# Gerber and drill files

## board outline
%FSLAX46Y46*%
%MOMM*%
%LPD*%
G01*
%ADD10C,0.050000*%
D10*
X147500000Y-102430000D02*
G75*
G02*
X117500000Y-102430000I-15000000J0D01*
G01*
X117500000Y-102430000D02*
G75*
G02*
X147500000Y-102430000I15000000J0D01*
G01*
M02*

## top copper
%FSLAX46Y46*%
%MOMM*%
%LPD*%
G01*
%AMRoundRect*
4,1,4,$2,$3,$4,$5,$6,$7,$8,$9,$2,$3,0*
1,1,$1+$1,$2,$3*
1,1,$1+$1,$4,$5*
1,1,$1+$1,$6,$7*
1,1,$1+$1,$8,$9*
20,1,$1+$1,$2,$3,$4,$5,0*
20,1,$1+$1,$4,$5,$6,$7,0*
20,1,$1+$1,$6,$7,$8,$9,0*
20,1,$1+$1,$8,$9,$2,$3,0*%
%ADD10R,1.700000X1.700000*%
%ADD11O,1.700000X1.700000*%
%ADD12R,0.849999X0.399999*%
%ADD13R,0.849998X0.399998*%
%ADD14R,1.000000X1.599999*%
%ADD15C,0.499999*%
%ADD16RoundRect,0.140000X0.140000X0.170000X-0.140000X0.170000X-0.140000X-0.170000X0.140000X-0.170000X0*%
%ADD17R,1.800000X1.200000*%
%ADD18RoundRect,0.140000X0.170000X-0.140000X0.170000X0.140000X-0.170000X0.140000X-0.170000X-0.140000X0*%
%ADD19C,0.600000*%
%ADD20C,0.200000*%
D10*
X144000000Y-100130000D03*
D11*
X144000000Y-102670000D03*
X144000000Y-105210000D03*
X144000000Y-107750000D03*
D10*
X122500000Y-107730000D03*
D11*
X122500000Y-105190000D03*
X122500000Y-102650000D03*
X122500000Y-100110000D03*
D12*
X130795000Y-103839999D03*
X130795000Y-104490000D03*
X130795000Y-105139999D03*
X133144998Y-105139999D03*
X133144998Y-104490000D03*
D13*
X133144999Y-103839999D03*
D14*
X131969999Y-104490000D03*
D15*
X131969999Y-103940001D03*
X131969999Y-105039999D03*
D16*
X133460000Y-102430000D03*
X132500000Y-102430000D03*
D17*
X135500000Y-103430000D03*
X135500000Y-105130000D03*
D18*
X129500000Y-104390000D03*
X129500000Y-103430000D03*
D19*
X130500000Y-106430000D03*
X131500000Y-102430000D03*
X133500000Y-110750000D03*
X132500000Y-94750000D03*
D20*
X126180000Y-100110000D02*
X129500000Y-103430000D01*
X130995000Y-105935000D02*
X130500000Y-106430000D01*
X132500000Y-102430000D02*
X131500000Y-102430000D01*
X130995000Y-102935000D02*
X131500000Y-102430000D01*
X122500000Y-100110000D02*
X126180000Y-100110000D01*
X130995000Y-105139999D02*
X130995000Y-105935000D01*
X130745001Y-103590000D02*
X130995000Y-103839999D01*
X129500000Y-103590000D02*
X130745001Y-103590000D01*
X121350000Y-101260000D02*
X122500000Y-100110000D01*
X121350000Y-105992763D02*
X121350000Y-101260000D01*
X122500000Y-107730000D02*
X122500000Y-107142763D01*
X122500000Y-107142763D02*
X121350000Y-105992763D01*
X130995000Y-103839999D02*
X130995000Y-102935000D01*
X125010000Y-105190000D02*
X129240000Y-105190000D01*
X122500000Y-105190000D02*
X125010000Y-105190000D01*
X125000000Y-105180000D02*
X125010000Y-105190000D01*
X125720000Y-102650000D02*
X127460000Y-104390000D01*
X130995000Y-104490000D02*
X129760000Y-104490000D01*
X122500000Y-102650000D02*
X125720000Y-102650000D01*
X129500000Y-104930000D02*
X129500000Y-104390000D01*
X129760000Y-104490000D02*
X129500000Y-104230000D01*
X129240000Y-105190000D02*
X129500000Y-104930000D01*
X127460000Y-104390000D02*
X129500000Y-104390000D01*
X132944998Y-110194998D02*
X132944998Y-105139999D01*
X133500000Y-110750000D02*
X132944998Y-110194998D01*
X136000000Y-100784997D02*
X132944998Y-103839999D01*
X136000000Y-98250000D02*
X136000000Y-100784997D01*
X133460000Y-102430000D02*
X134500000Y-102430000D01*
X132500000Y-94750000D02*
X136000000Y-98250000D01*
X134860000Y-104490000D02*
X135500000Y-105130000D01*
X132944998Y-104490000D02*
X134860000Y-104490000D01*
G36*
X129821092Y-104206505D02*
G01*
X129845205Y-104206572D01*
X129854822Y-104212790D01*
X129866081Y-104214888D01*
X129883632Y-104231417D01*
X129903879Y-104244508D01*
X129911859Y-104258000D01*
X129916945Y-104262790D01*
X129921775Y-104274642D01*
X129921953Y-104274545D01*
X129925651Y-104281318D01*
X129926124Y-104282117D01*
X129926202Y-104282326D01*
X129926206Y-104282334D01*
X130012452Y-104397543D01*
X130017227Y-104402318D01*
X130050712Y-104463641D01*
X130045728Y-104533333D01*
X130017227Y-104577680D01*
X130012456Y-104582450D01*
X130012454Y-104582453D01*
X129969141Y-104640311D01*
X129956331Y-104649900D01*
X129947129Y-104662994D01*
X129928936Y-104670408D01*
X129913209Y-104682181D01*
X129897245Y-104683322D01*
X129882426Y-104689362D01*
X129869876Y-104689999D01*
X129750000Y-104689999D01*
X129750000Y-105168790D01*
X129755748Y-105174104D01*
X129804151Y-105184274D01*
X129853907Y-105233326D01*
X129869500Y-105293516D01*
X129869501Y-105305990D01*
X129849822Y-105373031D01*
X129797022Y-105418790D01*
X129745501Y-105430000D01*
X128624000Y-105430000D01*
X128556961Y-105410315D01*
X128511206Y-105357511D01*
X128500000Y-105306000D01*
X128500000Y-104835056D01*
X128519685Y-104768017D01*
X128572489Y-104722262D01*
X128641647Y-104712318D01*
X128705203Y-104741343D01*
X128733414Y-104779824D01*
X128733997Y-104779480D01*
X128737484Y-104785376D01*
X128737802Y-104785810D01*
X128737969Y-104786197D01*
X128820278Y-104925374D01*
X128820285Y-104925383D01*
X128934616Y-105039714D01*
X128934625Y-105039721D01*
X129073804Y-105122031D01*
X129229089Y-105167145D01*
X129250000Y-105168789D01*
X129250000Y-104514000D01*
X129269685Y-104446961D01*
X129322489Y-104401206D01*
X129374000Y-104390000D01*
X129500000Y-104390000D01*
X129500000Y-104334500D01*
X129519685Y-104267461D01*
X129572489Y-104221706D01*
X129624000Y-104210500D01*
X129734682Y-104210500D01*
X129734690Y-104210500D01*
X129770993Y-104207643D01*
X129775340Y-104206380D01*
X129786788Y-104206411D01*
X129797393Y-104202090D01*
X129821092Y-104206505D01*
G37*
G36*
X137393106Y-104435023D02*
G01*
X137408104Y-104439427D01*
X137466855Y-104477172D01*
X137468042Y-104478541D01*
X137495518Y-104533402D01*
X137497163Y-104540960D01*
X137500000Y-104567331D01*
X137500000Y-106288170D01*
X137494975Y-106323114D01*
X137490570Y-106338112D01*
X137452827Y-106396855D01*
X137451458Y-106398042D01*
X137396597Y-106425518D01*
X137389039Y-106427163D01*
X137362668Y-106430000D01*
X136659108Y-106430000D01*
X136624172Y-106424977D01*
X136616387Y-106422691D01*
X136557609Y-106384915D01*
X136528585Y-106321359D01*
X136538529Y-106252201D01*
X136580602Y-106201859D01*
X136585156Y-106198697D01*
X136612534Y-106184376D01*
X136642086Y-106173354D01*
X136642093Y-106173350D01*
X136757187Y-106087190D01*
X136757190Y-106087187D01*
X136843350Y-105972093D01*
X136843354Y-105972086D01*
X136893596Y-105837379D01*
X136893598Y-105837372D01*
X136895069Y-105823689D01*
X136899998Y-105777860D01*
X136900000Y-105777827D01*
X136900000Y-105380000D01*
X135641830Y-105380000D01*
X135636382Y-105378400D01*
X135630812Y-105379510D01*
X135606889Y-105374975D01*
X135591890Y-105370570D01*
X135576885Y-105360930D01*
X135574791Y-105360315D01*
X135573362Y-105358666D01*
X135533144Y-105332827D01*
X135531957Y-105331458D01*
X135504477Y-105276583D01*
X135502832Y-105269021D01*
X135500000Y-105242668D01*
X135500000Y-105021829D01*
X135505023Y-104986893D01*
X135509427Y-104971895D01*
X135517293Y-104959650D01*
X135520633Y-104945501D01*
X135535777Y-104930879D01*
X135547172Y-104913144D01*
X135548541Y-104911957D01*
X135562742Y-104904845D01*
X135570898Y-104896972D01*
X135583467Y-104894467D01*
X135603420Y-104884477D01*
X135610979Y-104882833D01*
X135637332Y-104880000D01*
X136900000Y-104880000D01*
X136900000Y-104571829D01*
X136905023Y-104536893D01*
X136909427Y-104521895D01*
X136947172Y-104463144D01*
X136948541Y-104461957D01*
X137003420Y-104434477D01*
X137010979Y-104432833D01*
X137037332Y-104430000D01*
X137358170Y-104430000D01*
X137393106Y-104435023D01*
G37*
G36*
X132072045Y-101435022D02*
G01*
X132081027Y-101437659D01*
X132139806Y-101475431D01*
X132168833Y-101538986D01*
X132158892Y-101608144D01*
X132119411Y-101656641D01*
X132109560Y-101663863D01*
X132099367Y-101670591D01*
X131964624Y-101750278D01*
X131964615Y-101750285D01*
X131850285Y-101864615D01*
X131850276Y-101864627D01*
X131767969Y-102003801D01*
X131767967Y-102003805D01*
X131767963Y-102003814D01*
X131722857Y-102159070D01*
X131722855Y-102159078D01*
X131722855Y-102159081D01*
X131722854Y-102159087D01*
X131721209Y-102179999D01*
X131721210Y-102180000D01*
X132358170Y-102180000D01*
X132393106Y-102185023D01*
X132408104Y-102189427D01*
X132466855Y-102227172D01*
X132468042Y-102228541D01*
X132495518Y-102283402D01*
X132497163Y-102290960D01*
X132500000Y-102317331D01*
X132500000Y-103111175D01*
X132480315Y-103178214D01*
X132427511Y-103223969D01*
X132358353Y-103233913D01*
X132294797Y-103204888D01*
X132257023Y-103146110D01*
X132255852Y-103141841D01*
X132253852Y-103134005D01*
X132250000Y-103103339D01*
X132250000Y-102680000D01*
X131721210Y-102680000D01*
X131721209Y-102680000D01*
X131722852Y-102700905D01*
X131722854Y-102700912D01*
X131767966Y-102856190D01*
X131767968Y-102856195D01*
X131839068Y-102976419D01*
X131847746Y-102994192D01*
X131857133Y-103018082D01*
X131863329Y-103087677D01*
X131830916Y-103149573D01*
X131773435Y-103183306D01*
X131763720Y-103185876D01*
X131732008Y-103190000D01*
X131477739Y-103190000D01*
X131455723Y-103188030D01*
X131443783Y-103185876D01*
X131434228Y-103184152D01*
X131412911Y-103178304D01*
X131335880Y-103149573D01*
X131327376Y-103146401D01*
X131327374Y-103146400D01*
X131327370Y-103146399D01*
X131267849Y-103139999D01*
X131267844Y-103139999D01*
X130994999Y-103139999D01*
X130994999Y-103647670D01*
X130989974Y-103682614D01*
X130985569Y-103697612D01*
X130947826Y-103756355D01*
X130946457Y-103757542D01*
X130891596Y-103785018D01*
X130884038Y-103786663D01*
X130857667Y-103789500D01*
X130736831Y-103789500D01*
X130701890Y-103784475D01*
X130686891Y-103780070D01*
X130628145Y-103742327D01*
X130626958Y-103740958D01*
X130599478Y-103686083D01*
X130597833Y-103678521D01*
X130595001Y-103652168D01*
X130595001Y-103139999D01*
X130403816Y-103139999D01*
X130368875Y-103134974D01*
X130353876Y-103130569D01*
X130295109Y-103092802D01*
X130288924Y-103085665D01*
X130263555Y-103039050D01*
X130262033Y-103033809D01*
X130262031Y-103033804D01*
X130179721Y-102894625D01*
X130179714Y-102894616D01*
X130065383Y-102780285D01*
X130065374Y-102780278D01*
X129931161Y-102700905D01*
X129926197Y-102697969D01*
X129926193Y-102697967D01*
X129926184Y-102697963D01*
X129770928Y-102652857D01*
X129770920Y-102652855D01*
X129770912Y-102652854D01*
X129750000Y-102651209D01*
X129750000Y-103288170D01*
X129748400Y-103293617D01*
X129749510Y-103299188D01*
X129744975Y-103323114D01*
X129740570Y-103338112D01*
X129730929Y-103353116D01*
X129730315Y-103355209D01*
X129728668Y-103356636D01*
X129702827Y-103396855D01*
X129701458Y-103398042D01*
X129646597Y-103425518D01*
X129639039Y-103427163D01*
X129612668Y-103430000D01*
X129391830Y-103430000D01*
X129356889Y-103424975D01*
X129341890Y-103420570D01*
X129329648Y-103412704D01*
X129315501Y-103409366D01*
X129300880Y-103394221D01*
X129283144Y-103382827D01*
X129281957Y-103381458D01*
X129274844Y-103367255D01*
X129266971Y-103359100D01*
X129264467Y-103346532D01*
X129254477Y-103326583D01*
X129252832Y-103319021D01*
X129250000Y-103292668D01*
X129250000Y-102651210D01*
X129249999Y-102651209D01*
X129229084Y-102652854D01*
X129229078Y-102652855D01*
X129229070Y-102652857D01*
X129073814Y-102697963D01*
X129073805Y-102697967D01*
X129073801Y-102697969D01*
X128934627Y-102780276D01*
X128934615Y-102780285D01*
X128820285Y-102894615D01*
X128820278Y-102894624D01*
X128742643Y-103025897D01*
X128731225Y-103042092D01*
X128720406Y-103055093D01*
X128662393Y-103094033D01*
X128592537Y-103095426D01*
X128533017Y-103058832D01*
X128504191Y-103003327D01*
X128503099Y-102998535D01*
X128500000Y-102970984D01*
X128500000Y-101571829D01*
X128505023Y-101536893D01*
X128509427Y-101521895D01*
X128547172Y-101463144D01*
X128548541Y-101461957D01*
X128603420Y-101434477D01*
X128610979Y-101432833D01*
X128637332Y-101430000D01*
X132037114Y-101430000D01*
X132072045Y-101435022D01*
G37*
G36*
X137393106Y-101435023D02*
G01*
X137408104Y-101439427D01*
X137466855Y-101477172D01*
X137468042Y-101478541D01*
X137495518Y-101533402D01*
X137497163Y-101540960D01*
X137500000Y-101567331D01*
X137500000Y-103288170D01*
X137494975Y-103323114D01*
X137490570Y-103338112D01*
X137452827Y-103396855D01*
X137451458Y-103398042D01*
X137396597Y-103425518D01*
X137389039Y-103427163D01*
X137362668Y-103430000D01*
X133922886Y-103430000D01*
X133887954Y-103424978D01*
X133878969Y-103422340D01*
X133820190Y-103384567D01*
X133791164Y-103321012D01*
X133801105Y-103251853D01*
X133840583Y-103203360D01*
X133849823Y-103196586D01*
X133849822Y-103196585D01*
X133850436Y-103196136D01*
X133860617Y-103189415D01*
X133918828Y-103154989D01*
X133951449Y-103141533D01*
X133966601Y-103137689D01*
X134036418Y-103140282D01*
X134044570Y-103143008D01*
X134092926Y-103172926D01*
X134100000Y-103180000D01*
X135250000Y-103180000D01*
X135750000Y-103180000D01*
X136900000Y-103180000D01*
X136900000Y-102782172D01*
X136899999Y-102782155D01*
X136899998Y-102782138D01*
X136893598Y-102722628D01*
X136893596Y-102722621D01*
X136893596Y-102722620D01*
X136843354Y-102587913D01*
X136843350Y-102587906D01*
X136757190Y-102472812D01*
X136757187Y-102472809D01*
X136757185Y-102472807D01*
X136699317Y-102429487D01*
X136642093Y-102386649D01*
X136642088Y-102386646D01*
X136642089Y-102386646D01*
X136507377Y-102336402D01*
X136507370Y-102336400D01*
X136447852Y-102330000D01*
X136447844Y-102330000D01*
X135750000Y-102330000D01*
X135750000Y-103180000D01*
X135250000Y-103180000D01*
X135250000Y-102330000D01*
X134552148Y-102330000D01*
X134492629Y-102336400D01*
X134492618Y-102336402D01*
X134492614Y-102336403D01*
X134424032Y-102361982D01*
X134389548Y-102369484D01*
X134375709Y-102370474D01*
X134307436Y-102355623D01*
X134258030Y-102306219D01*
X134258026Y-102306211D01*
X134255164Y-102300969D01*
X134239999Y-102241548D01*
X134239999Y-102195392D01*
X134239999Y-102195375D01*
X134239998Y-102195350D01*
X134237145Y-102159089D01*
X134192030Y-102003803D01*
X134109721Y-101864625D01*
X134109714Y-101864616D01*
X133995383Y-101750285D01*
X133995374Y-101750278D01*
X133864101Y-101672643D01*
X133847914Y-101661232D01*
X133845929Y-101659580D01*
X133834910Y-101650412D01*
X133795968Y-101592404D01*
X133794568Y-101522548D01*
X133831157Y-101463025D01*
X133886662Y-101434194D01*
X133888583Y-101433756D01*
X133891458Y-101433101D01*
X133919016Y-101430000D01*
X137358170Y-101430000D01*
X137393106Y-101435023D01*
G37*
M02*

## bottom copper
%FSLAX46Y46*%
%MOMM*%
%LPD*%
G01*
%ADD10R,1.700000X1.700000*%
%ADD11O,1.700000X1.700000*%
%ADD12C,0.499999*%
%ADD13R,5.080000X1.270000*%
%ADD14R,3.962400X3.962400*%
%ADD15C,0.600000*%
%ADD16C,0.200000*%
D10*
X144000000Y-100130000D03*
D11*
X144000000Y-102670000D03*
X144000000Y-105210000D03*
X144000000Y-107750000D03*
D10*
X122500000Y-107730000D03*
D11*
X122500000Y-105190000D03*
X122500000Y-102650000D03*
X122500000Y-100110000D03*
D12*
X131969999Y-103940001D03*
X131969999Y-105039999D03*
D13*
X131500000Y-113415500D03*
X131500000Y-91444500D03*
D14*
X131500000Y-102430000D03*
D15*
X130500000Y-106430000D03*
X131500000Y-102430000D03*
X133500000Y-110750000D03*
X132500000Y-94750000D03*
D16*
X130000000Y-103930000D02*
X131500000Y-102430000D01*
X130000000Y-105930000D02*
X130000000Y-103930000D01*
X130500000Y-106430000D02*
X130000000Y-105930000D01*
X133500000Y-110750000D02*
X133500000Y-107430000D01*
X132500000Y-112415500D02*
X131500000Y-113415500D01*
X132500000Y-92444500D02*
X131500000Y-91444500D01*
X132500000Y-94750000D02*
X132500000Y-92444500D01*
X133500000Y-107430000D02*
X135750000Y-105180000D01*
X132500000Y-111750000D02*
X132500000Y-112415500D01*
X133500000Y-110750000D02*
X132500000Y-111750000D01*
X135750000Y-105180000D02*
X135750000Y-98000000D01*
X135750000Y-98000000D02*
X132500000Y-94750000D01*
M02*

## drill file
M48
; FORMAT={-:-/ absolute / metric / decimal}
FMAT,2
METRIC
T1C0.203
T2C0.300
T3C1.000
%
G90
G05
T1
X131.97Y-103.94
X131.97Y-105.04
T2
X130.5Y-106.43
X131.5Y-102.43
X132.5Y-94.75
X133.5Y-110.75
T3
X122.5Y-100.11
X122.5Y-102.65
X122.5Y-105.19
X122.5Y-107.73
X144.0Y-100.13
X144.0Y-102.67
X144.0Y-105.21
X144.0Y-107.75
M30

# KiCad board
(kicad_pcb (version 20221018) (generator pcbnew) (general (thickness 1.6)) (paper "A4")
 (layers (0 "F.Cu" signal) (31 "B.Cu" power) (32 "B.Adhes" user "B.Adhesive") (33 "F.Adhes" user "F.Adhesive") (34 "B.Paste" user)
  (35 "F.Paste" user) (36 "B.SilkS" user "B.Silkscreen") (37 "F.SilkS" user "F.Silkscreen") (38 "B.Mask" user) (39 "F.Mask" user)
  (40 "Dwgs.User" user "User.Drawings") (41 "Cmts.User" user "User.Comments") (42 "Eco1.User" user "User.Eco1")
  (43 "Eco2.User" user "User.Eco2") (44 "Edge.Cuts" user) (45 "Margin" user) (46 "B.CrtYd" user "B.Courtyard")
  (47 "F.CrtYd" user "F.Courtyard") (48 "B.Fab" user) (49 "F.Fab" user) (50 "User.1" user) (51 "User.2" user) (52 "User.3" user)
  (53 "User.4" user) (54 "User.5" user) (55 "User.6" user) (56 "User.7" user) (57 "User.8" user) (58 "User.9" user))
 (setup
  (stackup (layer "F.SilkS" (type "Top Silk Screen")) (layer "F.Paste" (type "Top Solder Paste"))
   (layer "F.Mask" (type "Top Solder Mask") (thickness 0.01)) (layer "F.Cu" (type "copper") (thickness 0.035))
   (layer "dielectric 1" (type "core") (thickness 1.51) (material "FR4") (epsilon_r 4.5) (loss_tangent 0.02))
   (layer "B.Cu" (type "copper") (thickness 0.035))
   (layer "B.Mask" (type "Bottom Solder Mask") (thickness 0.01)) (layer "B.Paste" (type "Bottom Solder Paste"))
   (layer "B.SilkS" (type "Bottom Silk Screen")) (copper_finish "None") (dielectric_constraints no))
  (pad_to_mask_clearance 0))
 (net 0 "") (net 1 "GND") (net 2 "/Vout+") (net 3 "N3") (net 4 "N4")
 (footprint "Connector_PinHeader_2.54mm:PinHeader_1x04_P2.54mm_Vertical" (layer "F.Cu") (at 144 100.13)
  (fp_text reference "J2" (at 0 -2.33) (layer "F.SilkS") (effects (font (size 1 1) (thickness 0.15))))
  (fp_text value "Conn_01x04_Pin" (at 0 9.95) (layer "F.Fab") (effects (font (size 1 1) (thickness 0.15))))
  (pad "1" thru_hole rect (at 0 0) (size 1.7 1.7) (drill 1) (layers "*.Cu" "*.Mask"))
  (pad "2" thru_hole oval (at 0 2.54) (size 1.7 1.7) (drill 1) (layers "*.Cu" "*.Mask"))
  (pad "3" thru_hole oval (at 0 5.08) (size 1.7 1.7) (drill 1) (layers "*.Cu" "*.Mask"))
  (pad "4" thru_hole oval (at 0 7.62) (size 1.7 1.7) (drill 1) (layers "*.Cu" "*.Mask")))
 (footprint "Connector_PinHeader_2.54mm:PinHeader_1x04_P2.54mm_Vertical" (layer "F.Cu") (at 122.5 107.73 180)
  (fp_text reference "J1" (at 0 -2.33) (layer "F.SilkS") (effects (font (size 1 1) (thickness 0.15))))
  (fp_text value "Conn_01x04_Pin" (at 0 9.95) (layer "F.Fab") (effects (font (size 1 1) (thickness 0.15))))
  (pad "1" thru_hole rect (at 0 0 180) (size 1.7 1.7) (drill 1) (layers "*.Cu" "*.Mask") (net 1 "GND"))
  (pad "2" thru_hole oval (at 0 2.54 180) (size 1.7 1.7) (drill 1) (layers "*.Cu" "*.Mask") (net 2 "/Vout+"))
  (pad "3" thru_hole oval (at 0 5.08 180) (size 1.7 1.7) (drill 1) (layers "*.Cu" "*.Mask") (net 2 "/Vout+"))
  (pad "4" thru_hole oval (at 0 7.62 180) (size 1.7 1.7) (drill 1) (layers "*.Cu" "*.Mask") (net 1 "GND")))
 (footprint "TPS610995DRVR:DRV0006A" (layer "F.Cu") (at 131.969999 104.49)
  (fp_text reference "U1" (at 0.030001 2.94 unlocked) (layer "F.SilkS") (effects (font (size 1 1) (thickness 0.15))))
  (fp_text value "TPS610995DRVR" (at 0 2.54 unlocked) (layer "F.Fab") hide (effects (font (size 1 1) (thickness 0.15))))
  (pad "1" smd rect (at -1.174999 -0.650001 90) (size 0.399999 0.849999) (layers "F.Cu" "F.Paste" "F.Mask") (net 1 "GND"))
  (pad "2" smd rect (at -1.174999 0 90) (size 0.399999 0.849999) (layers "F.Cu" "F.Paste" "F.Mask") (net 2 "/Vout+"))
  (pad "3" smd rect (at -1.174999 0.649999 90) (size 0.399999 0.849999) (layers "F.Cu" "F.Paste" "F.Mask") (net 1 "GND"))
  (pad "4" smd rect (at 1.174999 0.649999 90) (size 0.399999 0.849999) (layers "F.Cu" "F.Paste" "F.Mask") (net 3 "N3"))
  (pad "5" smd rect (at 1.174999 0 90) (size 0.399999 0.849999) (layers "F.Cu" "F.Paste" "F.Mask") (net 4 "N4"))
  (pad "6" smd rect (at 1.175 -0.650001 90) (size 0.399998 0.849998) (layers "F.Cu" "F.Paste" "F.Mask") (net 3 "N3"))
  (pad "7" smd rect (at 0 0) (size 1 1.599999) (layers "F.Cu" "F.Paste" "F.Mask") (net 1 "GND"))
  (pad "V" thru_hole circle (at 0 -0.549999) (size 0.499999 0.499999) (drill 0.2032) (layers "*.Cu" "*.Mask") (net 1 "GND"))
  (pad "V" thru_hole circle (at 0 0.549999) (size 0.499999 0.499999) (drill 0.2032) (layers "*.Cu" "*.Mask") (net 1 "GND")))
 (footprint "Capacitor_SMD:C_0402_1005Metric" (layer "F.Cu") (at 132.98 102.43 180)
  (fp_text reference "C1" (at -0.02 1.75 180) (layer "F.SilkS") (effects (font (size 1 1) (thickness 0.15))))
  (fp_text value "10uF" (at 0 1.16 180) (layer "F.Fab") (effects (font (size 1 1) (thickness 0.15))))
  (pad "1" smd roundrect (at -0.48 0 180) (size 0.56 0.62) (layers "F.Cu" "F.Paste" "F.Mask") (roundrect_rratio 0.25) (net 3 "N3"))
  (pad "2" smd roundrect (at 0.48 0 180) (size 0.56 0.62) (layers "F.Cu" "F.Paste" "F.Mask") (roundrect_rratio 0.25) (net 1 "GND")))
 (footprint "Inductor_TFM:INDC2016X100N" (layer "F.Cu") (at 135.5 104.28 -90)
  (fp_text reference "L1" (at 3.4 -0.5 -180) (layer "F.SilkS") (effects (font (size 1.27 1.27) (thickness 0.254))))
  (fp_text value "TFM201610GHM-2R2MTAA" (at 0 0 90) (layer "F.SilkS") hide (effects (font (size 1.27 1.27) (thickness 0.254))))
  (pad "1" smd rect (at -0.85 0 270) (size 1.2 1.8) (layers "F.Cu" "F.Paste" "F.Mask") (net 3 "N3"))
  (pad "2" smd rect (at 0.85 0 270) (size 1.2 1.8) (layers "F.Cu" "F.Paste" "F.Mask") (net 4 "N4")))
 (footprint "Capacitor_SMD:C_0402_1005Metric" (layer "F.Cu") (at 129.5 103.91 90)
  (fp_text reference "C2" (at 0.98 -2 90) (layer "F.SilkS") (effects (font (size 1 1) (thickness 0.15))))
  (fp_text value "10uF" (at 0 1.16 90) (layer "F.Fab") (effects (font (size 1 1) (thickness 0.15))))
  (pad "1" smd roundrect (at -0.48 0 90) (size 0.56 0.62) (layers "F.Cu" "F.Paste" "F.Mask") (roundrect_rratio 0.25) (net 2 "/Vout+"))
  (pad "2" smd roundrect (at 0.48 0 90) (size 0.56 0.62) (layers "F.Cu" "F.Paste" "F.Mask") (roundrect_rratio 0.25) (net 1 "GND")))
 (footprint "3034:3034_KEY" (layer "B.Cu") (at 132.1731 102.43 90)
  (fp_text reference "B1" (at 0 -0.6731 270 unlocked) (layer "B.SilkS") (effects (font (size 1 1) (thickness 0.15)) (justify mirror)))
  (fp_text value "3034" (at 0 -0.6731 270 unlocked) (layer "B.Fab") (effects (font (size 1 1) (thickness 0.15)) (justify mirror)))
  (pad "1" smd rect (at -10.9855 -0.6731 90) (size 1.27 5.08) (layers "B.Cu" "B.Paste" "B.Mask") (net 3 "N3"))
  (pad "2" smd rect (at 10.9855 -0.6731 90) (size 1.27 5.08) (layers "B.Cu" "B.Paste" "B.Mask") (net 3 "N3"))
  (pad "3" smd rect (at 0 -0.6731 90) (size 3.9624 3.9624) (layers "B.Cu" "B.Paste" "B.Mask") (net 1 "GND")))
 (gr_circle (center 132.5 102.43) (end 141.5 114.43) (stroke (width 0.05) (type default)) (fill none) (layer "Edge.Cuts"))
 (segment (start 126.18 100.11) (end 129.5 103.43) (width 0.2) (layer "F.Cu") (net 1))
 (segment (start 130.995 105.935) (end 130.5 106.43) (width 0.2) (layer "F.Cu") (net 1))
 (segment (start 132.5 102.43) (end 131.5 102.43) (width 0.2) (layer "F.Cu") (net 1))
 (segment (start 130.995 102.935) (end 131.5 102.43) (width 0.2) (layer "F.Cu") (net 1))
 (segment (start 122.5 100.11) (end 126.18 100.11) (width 0.2) (layer "F.Cu") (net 1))
 (segment (start 130.995 105.139999) (end 130.995 105.935) (width 0.2) (layer "F.Cu") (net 1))
 (segment (start 130.745001 103.59) (end 130.995 103.839999) (width 0.2) (layer "F.Cu") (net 1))
 (segment (start 129.5 103.59) (end 130.745001 103.59) (width 0.2) (layer "F.Cu") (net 1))
 (segment (start 121.35 101.26) (end 122.5 100.11) (width 0.2) (layer "F.Cu") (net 1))
 (segment (start 121.35 105.992763) (end 121.35 101.26) (width 0.2) (layer "F.Cu") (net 1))
 (segment (start 122.5 107.73) (end 122.5 107.142763) (width 0.2) (layer "F.Cu") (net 1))
 (segment (start 122.5 107.142763) (end 121.35 105.992763) (width 0.2) (layer "F.Cu") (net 1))
 (segment (start 130.995 103.839999) (end 130.995 102.935) (width 0.2) (layer "F.Cu") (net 1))
 (via (at 130.5 106.43) (size 0.6) (drill 0.3) (layers "F.Cu" "B.Cu") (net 1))
 (via (at 131.5 102.43) (size 0.6) (drill 0.3) (layers "F.Cu" "B.Cu") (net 1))
 (segment (start 130 103.93) (end 131.5 102.43) (width 0.2) (layer "B.Cu") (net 1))
 (segment (start 130 105.93) (end 130 103.93) (width 0.2) (layer "B.Cu") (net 1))
 (segment (start 130.5 106.43) (end 130 105.93) (width 0.2) (layer "B.Cu") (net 1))
 (segment (start 125.01 105.19) (end 129.24 105.19) (width 0.2) (layer "F.Cu") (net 2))
 (segment (start 122.5 105.19) (end 125.01 105.19) (width 0.2) (layer "F.Cu") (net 2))
 (segment (start 125 105.18) (end 125.01 105.19) (width 0.2) (layer "F.Cu") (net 2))
 (segment (start 125.72 102.65) (end 127.46 104.39) (width 0.2) (layer "F.Cu") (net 2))
 (segment (start 130.995 104.49) (end 129.76 104.49) (width 0.2) (layer "F.Cu") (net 2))
 (segment (start 122.5 102.65) (end 125.72 102.65) (width 0.2) (layer "F.Cu") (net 2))
 (segment (start 129.5 104.93) (end 129.5 104.39) (width 0.2) (layer "F.Cu") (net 2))
 (segment (start 129.76 104.49) (end 129.5 104.23) (width 0.2) (layer "F.Cu") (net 2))
 (segment (start 129.24 105.19) (end 129.5 104.93) (width 0.2) (layer "F.Cu") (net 2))
 (segment (start 127.46 104.39) (end 129.5 104.39) (width 0.2) (layer "F.Cu") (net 2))
 (segment (start 132.944998 110.194998) (end 132.944998 105.139999) (width 0.2) (layer "F.Cu") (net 3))
 (segment (start 133.5 110.75) (end 132.944998 110.194998) (width 0.2) (layer "F.Cu") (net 3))
 (segment (start 136 100.784997) (end 132.944998 103.839999) (width 0.2) (layer "F.Cu") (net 3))
 (segment (start 136 98.25) (end 136 100.784997) (width 0.2) (layer "F.Cu") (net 3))
 (segment (start 133.46 102.43) (end 134.5 102.43) (width 0.2) (layer "F.Cu") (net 3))
 (segment (start 132.5 94.75) (end 136 98.25) (width 0.2) (layer "F.Cu") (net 3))
 (via (at 133.5 110.75) (size 0.6) (drill 0.3) (layers "F.Cu" "B.Cu") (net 3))
 (via (at 132.5 94.75) (size 0.6) (drill 0.3) (layers "F.Cu" "B.Cu") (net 3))
 (segment (start 133.5 110.75) (end 133.5 107.43) (width 0.2) (layer "B.Cu") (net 3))
 (segment (start 132.5 112.4155) (end 131.5 113.4155) (width 0.2) (layer "B.Cu") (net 3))
 (segment (start 132.5 92.4445) (end 131.5 91.4445) (width 0.2) (layer "B.Cu") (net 3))
 (segment (start 132.5 94.75) (end 132.5 92.4445) (width 0.2) (layer "B.Cu") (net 3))
 (segment (start 133.5 107.43) (end 135.75 105.18) (width 0.2) (layer "B.Cu") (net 3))
 (segment (start 132.5 111.75) (end 132.5 112.4155) (width 0.2) (layer "B.Cu") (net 3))
 (segment (start 133.5 110.75) (end 132.5 111.75) (width 0.2) (layer "B.Cu") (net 3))
 (segment (start 135.75 105.18) (end 135.75 98) (width 0.2) (layer "B.Cu") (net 3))
 (segment (start 135.75 98) (end 132.5 94.75) (width 0.2) (layer "B.Cu") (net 3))
 (segment (start 134.86 104.49) (end 135.5 105.13) (width 0.2) (layer "F.Cu") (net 4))
 (segment (start 132.944998 104.49) (end 134.86 104.49) (width 0.2) (layer "F.Cu") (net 4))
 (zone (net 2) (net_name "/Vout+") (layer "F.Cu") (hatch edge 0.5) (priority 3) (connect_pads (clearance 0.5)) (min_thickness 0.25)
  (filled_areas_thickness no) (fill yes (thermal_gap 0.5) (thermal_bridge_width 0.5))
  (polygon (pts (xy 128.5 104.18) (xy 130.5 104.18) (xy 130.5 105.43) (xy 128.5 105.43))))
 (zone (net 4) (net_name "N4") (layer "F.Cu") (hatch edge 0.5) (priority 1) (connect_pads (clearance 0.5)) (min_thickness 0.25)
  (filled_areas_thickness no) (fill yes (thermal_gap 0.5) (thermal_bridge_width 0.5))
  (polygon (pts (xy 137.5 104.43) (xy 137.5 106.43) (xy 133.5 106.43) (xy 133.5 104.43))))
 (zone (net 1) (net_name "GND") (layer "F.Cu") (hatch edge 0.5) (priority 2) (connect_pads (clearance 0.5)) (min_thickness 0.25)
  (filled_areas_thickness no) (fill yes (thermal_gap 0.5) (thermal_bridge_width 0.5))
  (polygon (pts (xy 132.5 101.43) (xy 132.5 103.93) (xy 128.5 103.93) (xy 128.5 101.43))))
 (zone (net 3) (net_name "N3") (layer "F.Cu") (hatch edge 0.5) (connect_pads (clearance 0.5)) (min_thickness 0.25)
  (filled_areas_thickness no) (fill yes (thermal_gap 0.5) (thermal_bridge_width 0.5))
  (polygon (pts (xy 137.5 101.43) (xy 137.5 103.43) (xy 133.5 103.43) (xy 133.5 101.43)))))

